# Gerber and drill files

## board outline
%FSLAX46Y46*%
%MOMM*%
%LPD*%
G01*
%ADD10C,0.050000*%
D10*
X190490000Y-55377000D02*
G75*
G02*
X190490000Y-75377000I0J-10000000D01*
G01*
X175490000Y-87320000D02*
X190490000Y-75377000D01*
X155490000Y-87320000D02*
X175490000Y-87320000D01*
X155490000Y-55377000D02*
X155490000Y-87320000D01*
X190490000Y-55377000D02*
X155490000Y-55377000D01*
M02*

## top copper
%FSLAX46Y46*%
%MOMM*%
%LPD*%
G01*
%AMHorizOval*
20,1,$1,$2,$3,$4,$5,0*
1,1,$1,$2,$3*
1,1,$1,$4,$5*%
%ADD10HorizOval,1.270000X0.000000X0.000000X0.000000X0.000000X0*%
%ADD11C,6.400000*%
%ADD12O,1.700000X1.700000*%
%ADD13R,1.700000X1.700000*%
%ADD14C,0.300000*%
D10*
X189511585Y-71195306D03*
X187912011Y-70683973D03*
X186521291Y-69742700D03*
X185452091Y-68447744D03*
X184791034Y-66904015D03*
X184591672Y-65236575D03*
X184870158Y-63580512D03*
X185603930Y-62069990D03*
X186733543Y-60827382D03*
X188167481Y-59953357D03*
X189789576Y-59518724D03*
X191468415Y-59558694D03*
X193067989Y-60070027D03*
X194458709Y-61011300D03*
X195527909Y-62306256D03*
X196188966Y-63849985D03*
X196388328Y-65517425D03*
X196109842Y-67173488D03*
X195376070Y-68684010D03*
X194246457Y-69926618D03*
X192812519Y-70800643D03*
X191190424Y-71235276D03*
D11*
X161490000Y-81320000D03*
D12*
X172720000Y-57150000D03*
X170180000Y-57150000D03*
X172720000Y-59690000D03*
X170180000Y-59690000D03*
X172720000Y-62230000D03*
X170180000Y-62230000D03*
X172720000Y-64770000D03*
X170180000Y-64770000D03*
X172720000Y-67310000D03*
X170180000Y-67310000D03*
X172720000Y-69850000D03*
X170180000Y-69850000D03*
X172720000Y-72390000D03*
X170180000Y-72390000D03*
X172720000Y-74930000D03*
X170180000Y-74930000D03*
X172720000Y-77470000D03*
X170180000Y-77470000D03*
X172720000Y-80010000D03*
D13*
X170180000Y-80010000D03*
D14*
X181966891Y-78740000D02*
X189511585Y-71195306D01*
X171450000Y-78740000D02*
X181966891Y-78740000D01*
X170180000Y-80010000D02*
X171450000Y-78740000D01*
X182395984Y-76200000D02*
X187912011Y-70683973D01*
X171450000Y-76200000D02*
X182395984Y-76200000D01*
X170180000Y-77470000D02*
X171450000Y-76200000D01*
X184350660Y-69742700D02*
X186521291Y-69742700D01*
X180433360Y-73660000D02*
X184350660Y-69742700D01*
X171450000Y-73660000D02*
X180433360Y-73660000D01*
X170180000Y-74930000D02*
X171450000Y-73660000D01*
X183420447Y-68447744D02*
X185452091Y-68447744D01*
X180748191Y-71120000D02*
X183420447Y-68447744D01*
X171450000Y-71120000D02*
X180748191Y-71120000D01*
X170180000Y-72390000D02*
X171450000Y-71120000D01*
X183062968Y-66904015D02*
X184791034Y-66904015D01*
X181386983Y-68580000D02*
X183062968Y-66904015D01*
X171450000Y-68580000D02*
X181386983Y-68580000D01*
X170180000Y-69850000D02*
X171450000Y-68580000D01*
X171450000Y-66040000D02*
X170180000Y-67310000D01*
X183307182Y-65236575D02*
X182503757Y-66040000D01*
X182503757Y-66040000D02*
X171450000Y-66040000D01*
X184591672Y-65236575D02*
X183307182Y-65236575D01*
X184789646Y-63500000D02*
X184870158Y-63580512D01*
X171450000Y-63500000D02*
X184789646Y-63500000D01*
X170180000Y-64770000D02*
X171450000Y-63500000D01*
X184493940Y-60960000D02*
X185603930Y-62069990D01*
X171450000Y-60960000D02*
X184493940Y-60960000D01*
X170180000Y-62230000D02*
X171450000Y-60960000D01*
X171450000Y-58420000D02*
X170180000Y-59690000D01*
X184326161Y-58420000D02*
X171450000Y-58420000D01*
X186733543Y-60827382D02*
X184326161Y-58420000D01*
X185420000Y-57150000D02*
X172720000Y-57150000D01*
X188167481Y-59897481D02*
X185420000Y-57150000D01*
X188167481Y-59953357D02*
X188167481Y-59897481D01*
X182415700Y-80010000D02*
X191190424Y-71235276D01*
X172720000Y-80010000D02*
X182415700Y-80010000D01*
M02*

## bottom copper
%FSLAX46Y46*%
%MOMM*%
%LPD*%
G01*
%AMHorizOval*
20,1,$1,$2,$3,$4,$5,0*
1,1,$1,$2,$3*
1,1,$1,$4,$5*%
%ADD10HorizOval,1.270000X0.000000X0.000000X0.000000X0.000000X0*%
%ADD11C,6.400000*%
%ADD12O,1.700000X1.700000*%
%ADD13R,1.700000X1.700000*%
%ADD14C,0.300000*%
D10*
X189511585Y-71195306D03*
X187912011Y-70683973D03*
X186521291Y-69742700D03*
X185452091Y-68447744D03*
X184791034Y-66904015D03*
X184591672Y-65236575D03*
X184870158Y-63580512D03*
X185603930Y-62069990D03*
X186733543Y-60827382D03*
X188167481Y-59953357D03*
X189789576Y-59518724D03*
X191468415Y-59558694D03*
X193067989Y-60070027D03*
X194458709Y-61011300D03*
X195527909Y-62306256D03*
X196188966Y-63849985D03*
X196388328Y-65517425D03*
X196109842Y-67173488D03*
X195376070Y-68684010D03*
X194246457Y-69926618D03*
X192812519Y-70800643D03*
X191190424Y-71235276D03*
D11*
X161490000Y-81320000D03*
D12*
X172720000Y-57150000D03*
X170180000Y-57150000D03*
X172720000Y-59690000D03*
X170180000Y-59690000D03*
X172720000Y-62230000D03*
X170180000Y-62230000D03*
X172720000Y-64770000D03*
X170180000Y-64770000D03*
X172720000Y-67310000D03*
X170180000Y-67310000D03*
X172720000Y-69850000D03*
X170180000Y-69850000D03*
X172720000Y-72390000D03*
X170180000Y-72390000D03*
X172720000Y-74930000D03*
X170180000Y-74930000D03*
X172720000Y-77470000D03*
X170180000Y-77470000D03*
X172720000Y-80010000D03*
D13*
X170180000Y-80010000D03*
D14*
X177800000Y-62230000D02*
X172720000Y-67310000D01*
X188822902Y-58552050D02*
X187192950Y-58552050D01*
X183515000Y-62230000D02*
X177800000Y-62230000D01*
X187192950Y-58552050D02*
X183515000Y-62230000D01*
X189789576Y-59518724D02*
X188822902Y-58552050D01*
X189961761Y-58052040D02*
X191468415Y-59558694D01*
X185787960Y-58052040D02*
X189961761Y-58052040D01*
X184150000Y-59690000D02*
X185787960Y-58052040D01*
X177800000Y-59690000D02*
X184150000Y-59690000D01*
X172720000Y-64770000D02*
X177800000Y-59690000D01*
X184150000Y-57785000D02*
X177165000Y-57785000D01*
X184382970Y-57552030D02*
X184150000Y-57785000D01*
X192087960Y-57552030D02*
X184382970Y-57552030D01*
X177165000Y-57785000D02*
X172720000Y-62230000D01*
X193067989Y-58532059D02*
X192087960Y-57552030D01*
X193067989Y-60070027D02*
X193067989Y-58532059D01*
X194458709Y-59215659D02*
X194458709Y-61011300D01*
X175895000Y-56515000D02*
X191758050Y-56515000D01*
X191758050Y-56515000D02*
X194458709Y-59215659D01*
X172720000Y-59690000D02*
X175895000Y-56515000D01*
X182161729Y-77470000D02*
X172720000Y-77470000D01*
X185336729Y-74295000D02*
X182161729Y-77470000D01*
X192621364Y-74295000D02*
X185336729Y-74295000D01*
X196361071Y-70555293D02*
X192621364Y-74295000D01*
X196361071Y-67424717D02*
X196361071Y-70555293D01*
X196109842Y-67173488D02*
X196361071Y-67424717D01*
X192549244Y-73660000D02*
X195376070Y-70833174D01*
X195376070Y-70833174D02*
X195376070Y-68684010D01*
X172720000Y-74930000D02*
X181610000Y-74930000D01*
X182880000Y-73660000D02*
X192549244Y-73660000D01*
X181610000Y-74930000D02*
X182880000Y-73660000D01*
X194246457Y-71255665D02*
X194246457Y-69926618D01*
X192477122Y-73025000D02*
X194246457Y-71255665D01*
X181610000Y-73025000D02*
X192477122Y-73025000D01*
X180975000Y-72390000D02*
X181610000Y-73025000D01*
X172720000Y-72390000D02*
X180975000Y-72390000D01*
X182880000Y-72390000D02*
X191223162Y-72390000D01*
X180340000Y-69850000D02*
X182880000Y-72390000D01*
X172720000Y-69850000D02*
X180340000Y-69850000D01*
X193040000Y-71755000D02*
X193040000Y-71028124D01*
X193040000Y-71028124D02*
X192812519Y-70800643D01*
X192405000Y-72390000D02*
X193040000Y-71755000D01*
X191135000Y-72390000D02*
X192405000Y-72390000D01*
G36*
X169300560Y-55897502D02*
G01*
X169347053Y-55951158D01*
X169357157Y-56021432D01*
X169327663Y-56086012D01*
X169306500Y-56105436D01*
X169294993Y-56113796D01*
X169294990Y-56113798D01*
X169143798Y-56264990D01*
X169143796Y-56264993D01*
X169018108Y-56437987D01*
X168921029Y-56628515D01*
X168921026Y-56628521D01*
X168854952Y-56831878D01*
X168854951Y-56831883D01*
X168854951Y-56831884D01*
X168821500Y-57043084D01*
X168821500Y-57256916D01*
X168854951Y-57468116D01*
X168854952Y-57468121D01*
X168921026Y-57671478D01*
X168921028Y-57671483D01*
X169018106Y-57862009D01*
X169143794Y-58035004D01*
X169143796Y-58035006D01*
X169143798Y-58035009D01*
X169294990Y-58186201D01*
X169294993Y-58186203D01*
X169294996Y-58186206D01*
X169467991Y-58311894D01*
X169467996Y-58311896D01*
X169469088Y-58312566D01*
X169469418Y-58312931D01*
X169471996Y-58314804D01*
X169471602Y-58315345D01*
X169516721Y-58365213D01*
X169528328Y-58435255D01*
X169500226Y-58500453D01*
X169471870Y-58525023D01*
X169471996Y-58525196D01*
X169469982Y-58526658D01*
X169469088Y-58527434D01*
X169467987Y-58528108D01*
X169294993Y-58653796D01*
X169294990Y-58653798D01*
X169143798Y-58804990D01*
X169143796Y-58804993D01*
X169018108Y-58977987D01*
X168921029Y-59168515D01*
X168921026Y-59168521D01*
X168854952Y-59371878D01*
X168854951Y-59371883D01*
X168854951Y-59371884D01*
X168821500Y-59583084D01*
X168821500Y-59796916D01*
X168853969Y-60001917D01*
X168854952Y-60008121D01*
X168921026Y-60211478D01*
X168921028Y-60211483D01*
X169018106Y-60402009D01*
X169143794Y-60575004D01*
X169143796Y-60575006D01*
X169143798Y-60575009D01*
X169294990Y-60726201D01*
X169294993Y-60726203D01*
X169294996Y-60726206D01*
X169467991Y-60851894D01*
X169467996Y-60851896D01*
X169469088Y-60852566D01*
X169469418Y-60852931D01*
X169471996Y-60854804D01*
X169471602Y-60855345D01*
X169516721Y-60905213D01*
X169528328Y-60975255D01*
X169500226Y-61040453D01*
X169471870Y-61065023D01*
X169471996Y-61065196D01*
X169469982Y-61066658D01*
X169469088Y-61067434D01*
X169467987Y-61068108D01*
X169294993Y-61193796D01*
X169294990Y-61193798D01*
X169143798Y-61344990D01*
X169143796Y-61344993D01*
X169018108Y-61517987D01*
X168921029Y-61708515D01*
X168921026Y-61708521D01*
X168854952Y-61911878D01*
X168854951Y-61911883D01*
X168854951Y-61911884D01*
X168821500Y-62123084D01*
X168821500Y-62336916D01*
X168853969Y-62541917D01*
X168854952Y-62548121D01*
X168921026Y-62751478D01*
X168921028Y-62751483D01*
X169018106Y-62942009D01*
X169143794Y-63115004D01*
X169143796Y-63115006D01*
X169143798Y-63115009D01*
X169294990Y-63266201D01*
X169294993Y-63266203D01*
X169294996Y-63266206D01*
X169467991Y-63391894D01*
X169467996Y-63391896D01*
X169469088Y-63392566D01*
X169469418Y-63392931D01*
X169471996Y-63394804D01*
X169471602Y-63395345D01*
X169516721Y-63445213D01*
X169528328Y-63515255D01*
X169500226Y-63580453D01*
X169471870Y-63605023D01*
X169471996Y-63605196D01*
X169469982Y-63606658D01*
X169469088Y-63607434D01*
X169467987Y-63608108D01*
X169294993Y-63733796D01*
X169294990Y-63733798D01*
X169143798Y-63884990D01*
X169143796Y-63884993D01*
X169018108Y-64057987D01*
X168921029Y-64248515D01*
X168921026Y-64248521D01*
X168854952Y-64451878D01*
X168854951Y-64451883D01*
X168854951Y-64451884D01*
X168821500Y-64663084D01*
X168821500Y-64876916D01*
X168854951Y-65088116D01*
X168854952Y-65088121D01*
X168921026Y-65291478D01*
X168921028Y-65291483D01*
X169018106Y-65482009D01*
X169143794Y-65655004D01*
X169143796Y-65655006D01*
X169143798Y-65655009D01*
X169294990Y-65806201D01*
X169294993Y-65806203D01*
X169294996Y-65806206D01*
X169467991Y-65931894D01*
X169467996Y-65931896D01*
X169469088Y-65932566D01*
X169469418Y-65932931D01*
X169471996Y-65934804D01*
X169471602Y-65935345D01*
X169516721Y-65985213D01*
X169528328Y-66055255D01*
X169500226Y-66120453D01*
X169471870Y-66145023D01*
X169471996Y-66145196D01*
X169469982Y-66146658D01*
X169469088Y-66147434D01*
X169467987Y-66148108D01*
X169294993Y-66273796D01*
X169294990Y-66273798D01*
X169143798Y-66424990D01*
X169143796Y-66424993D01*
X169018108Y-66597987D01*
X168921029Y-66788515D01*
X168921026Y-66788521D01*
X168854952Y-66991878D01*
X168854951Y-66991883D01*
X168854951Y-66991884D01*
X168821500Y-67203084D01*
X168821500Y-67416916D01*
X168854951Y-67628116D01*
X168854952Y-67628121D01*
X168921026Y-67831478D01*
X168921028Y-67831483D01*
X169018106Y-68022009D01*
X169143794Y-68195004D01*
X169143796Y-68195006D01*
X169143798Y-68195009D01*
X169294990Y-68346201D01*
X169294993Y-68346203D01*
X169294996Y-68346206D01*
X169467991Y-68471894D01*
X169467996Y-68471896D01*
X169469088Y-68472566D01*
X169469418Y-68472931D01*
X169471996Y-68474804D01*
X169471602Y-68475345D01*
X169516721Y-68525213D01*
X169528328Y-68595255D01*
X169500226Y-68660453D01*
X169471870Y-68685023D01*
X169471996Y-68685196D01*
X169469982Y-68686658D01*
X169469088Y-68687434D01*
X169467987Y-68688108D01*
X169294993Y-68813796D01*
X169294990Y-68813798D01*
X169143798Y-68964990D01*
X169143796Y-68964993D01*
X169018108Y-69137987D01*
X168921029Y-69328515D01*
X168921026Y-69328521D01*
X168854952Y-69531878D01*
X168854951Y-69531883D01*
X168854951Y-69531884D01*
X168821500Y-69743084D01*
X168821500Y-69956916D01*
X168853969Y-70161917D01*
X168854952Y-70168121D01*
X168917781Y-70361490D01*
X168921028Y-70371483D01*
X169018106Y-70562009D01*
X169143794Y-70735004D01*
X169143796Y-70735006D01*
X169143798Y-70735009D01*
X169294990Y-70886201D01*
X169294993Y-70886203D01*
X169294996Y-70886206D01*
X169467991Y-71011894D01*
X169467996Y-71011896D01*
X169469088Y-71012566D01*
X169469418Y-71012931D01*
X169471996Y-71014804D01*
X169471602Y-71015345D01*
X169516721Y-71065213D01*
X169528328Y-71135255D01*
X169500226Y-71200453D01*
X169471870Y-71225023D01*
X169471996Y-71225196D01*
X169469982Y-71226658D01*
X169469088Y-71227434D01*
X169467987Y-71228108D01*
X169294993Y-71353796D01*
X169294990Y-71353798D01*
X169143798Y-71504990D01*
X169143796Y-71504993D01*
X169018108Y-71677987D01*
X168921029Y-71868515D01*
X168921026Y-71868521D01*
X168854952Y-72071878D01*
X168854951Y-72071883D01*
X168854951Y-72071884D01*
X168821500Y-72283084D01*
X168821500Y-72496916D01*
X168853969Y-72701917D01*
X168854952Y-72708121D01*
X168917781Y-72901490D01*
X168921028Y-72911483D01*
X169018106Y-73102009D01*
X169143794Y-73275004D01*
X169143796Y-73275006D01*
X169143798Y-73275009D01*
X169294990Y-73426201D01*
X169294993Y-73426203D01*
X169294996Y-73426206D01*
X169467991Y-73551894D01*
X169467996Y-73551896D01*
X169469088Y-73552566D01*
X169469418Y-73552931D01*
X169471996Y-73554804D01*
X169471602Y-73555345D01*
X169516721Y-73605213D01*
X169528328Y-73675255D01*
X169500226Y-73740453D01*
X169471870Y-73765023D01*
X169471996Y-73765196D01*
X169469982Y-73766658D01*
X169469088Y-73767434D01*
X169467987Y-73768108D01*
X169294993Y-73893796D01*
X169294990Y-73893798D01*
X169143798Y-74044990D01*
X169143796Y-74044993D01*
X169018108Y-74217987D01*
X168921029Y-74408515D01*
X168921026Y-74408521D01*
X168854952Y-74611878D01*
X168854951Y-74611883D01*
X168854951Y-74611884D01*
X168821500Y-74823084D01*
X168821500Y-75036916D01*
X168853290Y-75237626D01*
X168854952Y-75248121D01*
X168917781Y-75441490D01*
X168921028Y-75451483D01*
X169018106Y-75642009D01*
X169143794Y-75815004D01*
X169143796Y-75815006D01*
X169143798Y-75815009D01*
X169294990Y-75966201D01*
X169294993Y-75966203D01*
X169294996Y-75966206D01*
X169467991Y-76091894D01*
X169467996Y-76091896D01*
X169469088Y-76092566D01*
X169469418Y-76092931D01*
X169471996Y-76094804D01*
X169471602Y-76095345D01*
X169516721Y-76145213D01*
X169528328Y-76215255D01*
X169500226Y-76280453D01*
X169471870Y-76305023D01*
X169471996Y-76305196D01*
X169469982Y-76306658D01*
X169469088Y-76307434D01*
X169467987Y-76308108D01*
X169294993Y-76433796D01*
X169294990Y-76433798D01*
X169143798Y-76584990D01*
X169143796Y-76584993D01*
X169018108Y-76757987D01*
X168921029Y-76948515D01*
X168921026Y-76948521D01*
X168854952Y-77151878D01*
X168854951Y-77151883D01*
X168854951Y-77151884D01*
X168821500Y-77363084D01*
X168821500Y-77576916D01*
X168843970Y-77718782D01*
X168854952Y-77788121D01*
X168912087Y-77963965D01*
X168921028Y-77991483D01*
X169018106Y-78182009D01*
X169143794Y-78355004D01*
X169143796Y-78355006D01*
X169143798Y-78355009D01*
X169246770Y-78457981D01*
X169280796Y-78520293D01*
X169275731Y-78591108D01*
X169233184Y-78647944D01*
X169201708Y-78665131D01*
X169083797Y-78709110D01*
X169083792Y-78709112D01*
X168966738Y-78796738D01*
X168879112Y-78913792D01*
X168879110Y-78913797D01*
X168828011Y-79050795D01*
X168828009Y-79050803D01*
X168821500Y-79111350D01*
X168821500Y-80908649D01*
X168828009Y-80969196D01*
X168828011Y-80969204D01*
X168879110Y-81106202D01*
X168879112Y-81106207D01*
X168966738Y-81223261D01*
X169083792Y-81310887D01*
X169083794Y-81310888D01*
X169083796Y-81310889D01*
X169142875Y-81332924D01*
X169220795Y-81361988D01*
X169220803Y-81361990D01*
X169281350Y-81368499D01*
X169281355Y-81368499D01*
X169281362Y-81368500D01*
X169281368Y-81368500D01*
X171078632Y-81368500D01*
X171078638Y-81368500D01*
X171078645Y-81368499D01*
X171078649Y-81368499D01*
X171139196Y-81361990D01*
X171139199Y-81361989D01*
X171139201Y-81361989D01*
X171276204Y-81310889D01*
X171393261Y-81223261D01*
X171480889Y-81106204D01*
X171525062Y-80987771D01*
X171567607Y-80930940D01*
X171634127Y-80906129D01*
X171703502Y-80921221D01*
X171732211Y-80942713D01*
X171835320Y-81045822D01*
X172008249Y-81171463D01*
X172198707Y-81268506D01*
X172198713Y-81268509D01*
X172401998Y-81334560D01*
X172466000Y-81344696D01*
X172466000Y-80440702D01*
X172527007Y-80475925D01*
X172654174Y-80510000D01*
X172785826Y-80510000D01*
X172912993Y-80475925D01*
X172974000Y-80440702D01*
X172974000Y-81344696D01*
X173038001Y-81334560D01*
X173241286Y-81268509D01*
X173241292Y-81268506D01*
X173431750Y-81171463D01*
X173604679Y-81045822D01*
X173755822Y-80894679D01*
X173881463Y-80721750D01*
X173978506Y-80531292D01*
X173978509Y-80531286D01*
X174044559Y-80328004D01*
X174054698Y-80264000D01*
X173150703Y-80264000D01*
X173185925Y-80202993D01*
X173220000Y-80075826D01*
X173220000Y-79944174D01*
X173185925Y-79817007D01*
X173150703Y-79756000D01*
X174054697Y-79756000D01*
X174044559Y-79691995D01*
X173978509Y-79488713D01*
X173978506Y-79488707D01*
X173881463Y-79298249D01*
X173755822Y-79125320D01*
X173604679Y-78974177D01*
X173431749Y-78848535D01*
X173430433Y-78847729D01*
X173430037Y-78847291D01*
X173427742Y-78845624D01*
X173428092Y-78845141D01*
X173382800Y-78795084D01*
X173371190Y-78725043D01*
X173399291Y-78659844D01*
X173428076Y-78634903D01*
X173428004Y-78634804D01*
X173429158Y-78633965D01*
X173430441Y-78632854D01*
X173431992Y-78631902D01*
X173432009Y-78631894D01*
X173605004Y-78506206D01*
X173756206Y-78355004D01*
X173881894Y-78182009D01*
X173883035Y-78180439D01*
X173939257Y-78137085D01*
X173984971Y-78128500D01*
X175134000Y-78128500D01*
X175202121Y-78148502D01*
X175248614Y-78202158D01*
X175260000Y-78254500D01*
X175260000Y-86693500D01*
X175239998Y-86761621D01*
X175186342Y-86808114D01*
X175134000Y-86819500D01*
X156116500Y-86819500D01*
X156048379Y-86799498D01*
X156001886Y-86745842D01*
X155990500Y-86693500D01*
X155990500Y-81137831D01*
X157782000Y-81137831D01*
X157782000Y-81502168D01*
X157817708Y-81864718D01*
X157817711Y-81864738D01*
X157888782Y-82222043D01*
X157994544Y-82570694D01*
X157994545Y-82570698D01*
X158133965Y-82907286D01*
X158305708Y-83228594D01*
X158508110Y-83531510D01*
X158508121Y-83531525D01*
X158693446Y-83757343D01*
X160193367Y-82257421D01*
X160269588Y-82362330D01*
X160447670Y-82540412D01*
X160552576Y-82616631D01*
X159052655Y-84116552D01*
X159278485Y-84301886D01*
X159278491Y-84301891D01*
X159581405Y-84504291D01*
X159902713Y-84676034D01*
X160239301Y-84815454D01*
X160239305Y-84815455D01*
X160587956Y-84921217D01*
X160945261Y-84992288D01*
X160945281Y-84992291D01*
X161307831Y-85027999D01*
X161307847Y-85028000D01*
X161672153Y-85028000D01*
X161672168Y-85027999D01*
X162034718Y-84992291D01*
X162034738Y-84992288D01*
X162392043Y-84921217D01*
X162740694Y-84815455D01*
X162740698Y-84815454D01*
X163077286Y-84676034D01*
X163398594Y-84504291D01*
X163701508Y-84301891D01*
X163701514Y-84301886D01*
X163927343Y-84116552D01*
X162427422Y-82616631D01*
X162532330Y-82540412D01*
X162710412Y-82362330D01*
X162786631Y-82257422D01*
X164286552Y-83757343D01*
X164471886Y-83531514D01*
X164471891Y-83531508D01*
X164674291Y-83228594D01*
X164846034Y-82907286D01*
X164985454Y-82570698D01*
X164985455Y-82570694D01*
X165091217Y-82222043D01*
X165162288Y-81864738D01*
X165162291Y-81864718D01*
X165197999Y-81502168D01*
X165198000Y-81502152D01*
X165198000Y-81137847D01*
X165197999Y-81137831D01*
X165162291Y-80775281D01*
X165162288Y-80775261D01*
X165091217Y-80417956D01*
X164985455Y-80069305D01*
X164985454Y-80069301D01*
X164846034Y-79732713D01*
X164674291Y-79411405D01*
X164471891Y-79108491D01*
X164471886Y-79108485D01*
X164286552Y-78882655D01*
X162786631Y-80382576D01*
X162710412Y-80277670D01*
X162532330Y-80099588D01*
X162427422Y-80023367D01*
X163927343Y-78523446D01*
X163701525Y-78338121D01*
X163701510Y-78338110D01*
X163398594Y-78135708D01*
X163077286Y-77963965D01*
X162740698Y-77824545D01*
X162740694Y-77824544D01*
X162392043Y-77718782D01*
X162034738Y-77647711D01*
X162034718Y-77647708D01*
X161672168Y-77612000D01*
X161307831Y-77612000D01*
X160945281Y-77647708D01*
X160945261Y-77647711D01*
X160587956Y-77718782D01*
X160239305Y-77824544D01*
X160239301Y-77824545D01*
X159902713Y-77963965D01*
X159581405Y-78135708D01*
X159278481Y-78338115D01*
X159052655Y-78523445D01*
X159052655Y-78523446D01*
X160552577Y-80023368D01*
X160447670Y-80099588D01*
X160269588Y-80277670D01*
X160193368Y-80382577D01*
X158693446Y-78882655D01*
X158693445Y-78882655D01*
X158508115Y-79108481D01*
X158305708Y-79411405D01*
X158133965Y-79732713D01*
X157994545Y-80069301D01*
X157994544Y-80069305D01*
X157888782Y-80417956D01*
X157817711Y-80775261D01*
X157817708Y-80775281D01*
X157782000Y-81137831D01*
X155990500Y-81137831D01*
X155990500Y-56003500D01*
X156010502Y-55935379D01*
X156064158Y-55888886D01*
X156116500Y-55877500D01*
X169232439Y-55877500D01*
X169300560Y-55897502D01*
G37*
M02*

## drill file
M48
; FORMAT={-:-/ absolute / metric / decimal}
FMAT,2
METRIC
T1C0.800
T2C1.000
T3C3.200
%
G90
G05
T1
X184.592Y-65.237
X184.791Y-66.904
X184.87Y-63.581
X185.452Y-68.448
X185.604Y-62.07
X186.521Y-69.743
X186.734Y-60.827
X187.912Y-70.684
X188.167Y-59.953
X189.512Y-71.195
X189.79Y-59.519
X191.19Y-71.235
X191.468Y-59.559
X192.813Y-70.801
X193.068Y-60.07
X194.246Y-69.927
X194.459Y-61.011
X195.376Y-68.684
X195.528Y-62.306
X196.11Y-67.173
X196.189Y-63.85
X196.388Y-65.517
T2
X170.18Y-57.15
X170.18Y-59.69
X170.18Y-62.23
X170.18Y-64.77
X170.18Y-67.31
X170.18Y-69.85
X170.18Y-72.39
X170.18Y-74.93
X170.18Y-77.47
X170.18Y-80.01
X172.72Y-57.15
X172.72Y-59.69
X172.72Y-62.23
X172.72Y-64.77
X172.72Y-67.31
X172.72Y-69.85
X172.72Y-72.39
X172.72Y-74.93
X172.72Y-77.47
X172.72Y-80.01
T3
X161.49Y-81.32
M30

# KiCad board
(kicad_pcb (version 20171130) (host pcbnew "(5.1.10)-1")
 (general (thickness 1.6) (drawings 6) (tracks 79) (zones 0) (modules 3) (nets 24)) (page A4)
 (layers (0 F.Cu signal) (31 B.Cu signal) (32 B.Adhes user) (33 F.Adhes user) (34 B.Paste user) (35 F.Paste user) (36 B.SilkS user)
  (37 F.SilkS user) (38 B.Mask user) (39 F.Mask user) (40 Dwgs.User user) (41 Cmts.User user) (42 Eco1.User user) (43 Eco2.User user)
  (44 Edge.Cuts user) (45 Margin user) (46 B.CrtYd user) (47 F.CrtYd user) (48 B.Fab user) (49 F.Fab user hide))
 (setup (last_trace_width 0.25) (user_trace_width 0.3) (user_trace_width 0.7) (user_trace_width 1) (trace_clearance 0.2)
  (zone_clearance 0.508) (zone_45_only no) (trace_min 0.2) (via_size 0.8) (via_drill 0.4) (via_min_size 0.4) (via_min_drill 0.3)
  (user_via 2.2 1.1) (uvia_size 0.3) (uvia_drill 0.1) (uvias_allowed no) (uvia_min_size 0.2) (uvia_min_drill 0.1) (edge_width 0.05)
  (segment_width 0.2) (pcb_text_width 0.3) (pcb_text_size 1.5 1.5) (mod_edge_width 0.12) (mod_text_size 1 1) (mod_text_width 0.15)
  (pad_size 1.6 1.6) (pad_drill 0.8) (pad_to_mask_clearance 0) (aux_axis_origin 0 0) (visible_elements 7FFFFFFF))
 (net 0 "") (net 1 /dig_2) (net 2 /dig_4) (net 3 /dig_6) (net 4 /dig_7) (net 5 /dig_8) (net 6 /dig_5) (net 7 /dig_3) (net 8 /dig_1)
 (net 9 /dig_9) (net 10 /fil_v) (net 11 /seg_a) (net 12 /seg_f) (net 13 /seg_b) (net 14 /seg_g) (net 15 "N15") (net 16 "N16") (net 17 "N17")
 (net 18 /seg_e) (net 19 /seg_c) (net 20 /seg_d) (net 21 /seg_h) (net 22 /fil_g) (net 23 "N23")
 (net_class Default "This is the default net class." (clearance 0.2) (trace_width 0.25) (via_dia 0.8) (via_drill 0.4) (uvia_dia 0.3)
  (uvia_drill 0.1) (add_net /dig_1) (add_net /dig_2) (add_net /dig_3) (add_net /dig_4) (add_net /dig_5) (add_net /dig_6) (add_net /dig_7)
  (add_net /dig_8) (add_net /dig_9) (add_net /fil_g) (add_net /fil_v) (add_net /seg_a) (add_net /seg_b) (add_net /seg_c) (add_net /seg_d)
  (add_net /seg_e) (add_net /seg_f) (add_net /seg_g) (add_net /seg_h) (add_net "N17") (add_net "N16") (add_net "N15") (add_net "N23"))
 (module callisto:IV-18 (layer F.Cu) (at 190.49 65.377 15)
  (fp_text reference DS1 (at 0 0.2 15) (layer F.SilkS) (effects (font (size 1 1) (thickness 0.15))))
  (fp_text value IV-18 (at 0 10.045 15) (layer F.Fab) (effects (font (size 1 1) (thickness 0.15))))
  (pad 22 thru_hole oval (at -2.450965 5.36682 15) (size 1.27 1.27) (drill 0.8) (layers *.Cu *.Mask) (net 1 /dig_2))
  (pad 21 thru_hole oval (at -3.863692 4.45891 15) (size 1.27 1.27) (drill 0.8) (layers *.Cu *.Mask) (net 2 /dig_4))
  (pad 20 thru_hole oval (at -4.963405 3.189765 15) (size 1.27 1.27) (drill 0.8) (layers *.Cu *.Mask) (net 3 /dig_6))
  (pad 19 thru_hole oval (at -5.661013 1.662204 15) (size 1.27 1.27) (drill 0.8) (layers *.Cu *.Mask) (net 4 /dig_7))
  (pad 18 thru_hole oval (at -5.899999 -0.000018 15) (size 1.27 1.27) (drill 0.8) (layers *.Cu *.Mask) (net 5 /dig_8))
  (pad 17 thru_hole oval (at -5.661003 -1.66224 15) (size 1.27 1.27) (drill 0.8) (layers *.Cu *.Mask) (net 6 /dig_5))
  (pad 16 thru_hole oval (at -4.963385 -3.189796 15) (size 1.27 1.27) (drill 0.8) (layers *.Cu *.Mask) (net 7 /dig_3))
  (pad 15 thru_hole oval (at -3.863664 -4.458934 15) (size 1.27 1.27) (drill 0.8) (layers *.Cu *.Mask) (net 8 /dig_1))
  (pad 14 thru_hole oval (at -2.450931 -5.366836 15) (size 1.27 1.27) (drill 0.8) (layers *.Cu *.Mask) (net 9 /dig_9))
  (pad 13 thru_hole oval (at -0.839639 -5.839949 15) (size 1.27 1.27) (drill 0.8) (layers *.Cu *.Mask) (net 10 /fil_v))
  (pad 12 thru_hole oval (at 0.839676 -5.839943 15) (size 1.27 1.27) (drill 0.8) (layers *.Cu *.Mask) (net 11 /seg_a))
  (pad 11 thru_hole oval (at 2.450965 -5.36682 15) (size 1.27 1.27) (drill 0.8) (layers *.Cu *.Mask) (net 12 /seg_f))
  (pad 10 thru_hole oval (at 3.863692 -4.45891 15) (size 1.27 1.27) (drill 0.8) (layers *.Cu *.Mask) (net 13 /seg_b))
  (pad 9 thru_hole oval (at 4.963405 -3.189765 15) (size 1.27 1.27) (drill 0.8) (layers *.Cu *.Mask) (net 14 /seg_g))
  (pad 8 thru_hole oval (at 5.661013 -1.662204 15) (size 1.27 1.27) (drill 0.8) (layers *.Cu *.Mask) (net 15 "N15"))
  (pad 7 thru_hole oval (at 5.899999 0.000018 15) (size 1.27 1.27) (drill 0.8) (layers *.Cu *.Mask) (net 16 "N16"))
  (pad 6 thru_hole oval (at 5.661003 1.66224 15) (size 1.27 1.27) (drill 0.8) (layers *.Cu *.Mask) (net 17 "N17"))
  (pad 5 thru_hole oval (at 4.963385 3.189796 15) (size 1.27 1.27) (drill 0.8) (layers *.Cu *.Mask) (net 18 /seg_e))
  (pad 4 thru_hole oval (at 3.863664 4.458934 15) (size 1.27 1.27) (drill 0.8) (layers *.Cu *.Mask) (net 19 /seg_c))
  (pad 3 thru_hole oval (at 2.450931 5.366836 15) (size 1.27 1.27) (drill 0.8) (layers *.Cu *.Mask) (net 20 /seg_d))
  (pad 2 thru_hole oval (at 0.839639 5.839949 15) (size 1.27 1.27) (drill 0.8) (layers *.Cu *.Mask) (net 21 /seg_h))
  (pad 1 thru_hole oval (at -0.839676 5.839943 15) (size 1.27 1.27) (drill 0.8) (layers *.Cu *.Mask) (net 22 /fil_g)))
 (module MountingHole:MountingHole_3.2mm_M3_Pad (layer F.Cu) (at 161.49 81.32)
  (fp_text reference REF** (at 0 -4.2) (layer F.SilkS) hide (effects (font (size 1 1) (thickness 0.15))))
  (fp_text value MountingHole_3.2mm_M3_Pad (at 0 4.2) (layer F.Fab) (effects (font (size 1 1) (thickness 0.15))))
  (pad 1 thru_hole circle (at 0 0) (size 6.4 6.4) (drill 3.2) (layers *.Cu *.Mask) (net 22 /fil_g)))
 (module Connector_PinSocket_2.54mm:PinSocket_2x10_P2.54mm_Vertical (layer F.Cu) (at 170.18 80.01 180)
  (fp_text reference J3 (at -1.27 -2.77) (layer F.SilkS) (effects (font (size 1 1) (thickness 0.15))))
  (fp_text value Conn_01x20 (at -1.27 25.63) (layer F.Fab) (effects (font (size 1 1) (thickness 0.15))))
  (pad 20 thru_hole oval (at -2.54 22.86 180) (size 1.7 1.7) (drill 1) (layers *.Cu *.Mask) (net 10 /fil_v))
  (pad 19 thru_hole oval (at 0 22.86 180) (size 1.7 1.7) (drill 1) (layers *.Cu *.Mask) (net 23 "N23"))
  (pad 18 thru_hole oval (at -2.54 20.32 180) (size 1.7 1.7) (drill 1) (layers *.Cu *.Mask) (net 14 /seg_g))
  (pad 17 thru_hole oval (at 0 20.32 180) (size 1.7 1.7) (drill 1) (layers *.Cu *.Mask) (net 9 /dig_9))
  (pad 16 thru_hole oval (at -2.54 17.78 180) (size 1.7 1.7) (drill 1) (layers *.Cu *.Mask) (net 13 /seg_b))
  (pad 15 thru_hole oval (at 0 17.78 180) (size 1.7 1.7) (drill 1) (layers *.Cu *.Mask) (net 8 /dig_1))
  (pad 14 thru_hole oval (at -2.54 15.24 180) (size 1.7 1.7) (drill 1) (layers *.Cu *.Mask) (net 12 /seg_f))
  (pad 13 thru_hole oval (at 0 15.24 180) (size 1.7 1.7) (drill 1) (layers *.Cu *.Mask) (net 7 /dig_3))
  (pad 12 thru_hole oval (at -2.54 12.7 180) (size 1.7 1.7) (drill 1) (layers *.Cu *.Mask) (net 11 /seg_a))
  (pad 11 thru_hole oval (at 0 12.7 180) (size 1.7 1.7) (drill 1) (layers *.Cu *.Mask) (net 6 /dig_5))
  (pad 10 thru_hole oval (at -2.54 10.16 180) (size 1.7 1.7) (drill 1) (layers *.Cu *.Mask) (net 21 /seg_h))
  (pad 9 thru_hole oval (at 0 10.16 180) (size 1.7 1.7) (drill 1) (layers *.Cu *.Mask) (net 5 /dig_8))
  (pad 8 thru_hole oval (at -2.54 7.62 180) (size 1.7 1.7) (drill 1) (layers *.Cu *.Mask) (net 20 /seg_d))
  (pad 7 thru_hole oval (at 0 7.62 180) (size 1.7 1.7) (drill 1) (layers *.Cu *.Mask) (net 4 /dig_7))
  (pad 6 thru_hole oval (at -2.54 5.08 180) (size 1.7 1.7) (drill 1) (layers *.Cu *.Mask) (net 19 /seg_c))
  (pad 5 thru_hole oval (at 0 5.08 180) (size 1.7 1.7) (drill 1) (layers *.Cu *.Mask) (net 3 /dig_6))
  (pad 4 thru_hole oval (at -2.54 2.54 180) (size 1.7 1.7) (drill 1) (layers *.Cu *.Mask) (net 18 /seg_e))
  (pad 3 thru_hole oval (at 0 2.54 180) (size 1.7 1.7) (drill 1) (layers *.Cu *.Mask) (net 2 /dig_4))
  (pad 2 thru_hole oval (at -2.54 0 180) (size 1.7 1.7) (drill 1) (layers *.Cu *.Mask) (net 22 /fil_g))
  (pad 1 thru_hole rect (at 0 0 180) (size 1.7 1.7) (drill 1) (layers *.Cu *.Mask) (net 1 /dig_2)))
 (gr_arc (start 190.49 65.377) (end 190.49 75.377) (angle -180) (layer Edge.Cuts) (width 0.05))
 (gr_line (start 175.49 87.32) (end 190.49 75.377) (layer Edge.Cuts) (width 0.05))
 (gr_line (start 155.49 87.32) (end 175.49 87.32) (layer Edge.Cuts) (width 0.05))
 (gr_line (start 155.49 55.377) (end 155.49 87.32) (layer Edge.Cuts) (width 0.05))
 (gr_line (start 190.49 55.377) (end 155.49 55.377) (layer Edge.Cuts) (width 0.05))
 (segment (start 181.966891 78.74) (end 189.511585 71.195306) (width 0.3) (layer F.Cu) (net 1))
 (segment (start 171.45 78.74) (end 181.966891 78.74) (width 0.3) (layer F.Cu) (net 1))
 (segment (start 170.18 80.01) (end 171.45 78.74) (width 0.3) (layer F.Cu) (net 1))
 (segment (start 182.395984 76.2) (end 187.912011 70.683973) (width 0.3) (layer F.Cu) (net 2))
 (segment (start 171.45 76.2) (end 182.395984 76.2) (width 0.3) (layer F.Cu) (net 2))
 (segment (start 170.18 77.47) (end 171.45 76.2) (width 0.3) (layer F.Cu) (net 2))
 (segment (start 184.35066 69.7427) (end 186.521291 69.7427) (width 0.3) (layer F.Cu) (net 3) (status 20))
 (segment (start 180.43336 73.66) (end 184.35066 69.7427) (width 0.3) (layer F.Cu) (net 3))
 (segment (start 171.45 73.66) (end 180.43336 73.66) (width 0.3) (layer F.Cu) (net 3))
 (segment (start 170.18 74.93) (end 171.45 73.66) (width 0.3) (layer F.Cu) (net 3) (status 10))
 (segment (start 183.420447 68.447744) (end 185.452091 68.447744) (width 0.3) (layer F.Cu) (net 4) (status 20))
 (segment (start 180.748191 71.12) (end 183.420447 68.447744) (width 0.3) (layer F.Cu) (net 4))
 (segment (start 171.45 71.12) (end 180.748191 71.12) (width 0.3) (layer F.Cu) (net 4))
 (segment (start 170.18 72.39) (end 171.45 71.12) (width 0.3) (layer F.Cu) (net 4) (status 10))
 (segment (start 183.062968 66.904015) (end 184.791034 66.904015) (width 0.3) (layer F.Cu) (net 5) (status 20))
 (segment (start 181.386983 68.58) (end 183.062968 66.904015) (width 0.3) (layer F.Cu) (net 5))
 (segment (start 171.45 68.58) (end 181.386983 68.58) (width 0.3) (layer F.Cu) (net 5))
 (segment (start 170.18 69.85) (end 171.45 68.58) (width 0.3) (layer F.Cu) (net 5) (status 10))
 (segment (start 171.45 66.04) (end 170.18 67.31) (width 0.3) (layer F.Cu) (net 6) (status 20))
 (segment (start 183.307182 65.236575) (end 182.503757 66.04) (width 0.3) (layer F.Cu) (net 6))
 (segment (start 182.503757 66.04) (end 171.45 66.04) (width 0.3) (layer F.Cu) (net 6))
 (segment (start 184.591672 65.236575) (end 183.307182 65.236575) (width 0.3) (layer F.Cu) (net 6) (status 10))
 (segment (start 184.789646 63.5) (end 184.870158 63.580512) (width 0.3) (layer F.Cu) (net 7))
 (segment (start 171.45 63.5) (end 184.789646 63.5) (width 0.3) (layer F.Cu) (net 7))
 (segment (start 170.18 64.77) (end 171.45 63.5) (width 0.3) (layer F.Cu) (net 7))
 (segment (start 184.49394 60.96) (end 185.60393 62.06999) (width 0.3) (layer F.Cu) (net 8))
 (segment (start 171.45 60.96) (end 184.49394 60.96) (width 0.3) (layer F.Cu) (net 8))
 (segment (start 170.18 62.23) (end 171.45 60.96) (width 0.3) (layer F.Cu) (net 8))
 (segment (start 171.45 58.42) (end 170.18 59.69) (width 0.3) (layer F.Cu) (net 9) (status 20))
 (segment (start 184.326161 58.42) (end 171.45 58.42) (width 0.3) (layer F.Cu) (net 9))
 (segment (start 186.733543 60.827382) (end 184.326161 58.42) (width 0.3) (layer F.Cu) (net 9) (status 10))
 (segment (start 185.42 57.15) (end 172.72 57.15) (width 0.3) (layer F.Cu) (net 10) (status 20))
 (segment (start 188.167481 59.897481) (end 185.42 57.15) (width 0.3) (layer F.Cu) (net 10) (status 10))
 (segment (start 188.167481 59.953357) (end 188.167481 59.897481) (width 0.3) (layer F.Cu) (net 10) (status 30))
 (segment (start 177.8 62.23) (end 172.72 67.31) (width 0.3) (layer B.Cu) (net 11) (status 20))
 (segment (start 188.822902 58.55205) (end 187.19295 58.55205) (width 0.3) (layer B.Cu) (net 11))
 (segment (start 183.515 62.23) (end 177.8 62.23) (width 0.3) (layer B.Cu) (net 11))
 (segment (start 187.19295 58.55205) (end 183.515 62.23) (width 0.3) (layer B.Cu) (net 11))
 (segment (start 189.789576 59.518724) (end 188.822902 58.55205) (width 0.3) (layer B.Cu) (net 11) (status 10))
 (segment (start 189.961761 58.05204) (end 191.468415 59.558694) (width 0.3) (layer B.Cu) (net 12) (status 20))
 (segment (start 185.78796 58.05204) (end 189.961761 58.05204) (width 0.3) (layer B.Cu) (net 12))
 (segment (start 184.15 59.69) (end 185.78796 58.05204) (width 0.3) (layer B.Cu) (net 12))
 (segment (start 177.8 59.69) (end 184.15 59.69) (width 0.3) (layer B.Cu) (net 12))
 (segment (start 172.72 64.77) (end 177.8 59.69) (width 0.3) (layer B.Cu) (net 12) (status 10))
 (segment (start 184.15 57.785) (end 177.165 57.785) (width 0.3) (layer B.Cu) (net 13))
 (segment (start 184.38297 57.55203) (end 184.15 57.785) (width 0.3) (layer B.Cu) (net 13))
 (segment (start 192.08796 57.55203) (end 184.38297 57.55203) (width 0.3) (layer B.Cu) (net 13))
 (segment (start 177.165 57.785) (end 172.72 62.23) (width 0.3) (layer B.Cu) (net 13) (status 20))
 (segment (start 193.067989 58.532059) (end 192.08796 57.55203) (width 0.3) (layer B.Cu) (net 13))
 (segment (start 193.067989 60.070027) (end 193.067989 58.532059) (width 0.3) (layer B.Cu) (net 13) (status 10))
 (segment (start 194.458709 59.215659) (end 194.458709 61.0113) (width 0.3) (layer B.Cu) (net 14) (status 20))
 (segment (start 175.895 56.515) (end 191.75805 56.515) (width 0.3) (layer B.Cu) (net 14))
 (segment (start 191.75805 56.515) (end 194.458709 59.215659) (width 0.3) (layer B.Cu) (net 14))
 (segment (start 172.72 59.69) (end 175.895 56.515) (width 0.3) (layer B.Cu) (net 14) (status 10))
 (segment (start 182.161729 77.47) (end 172.72 77.47) (width 0.3) (layer B.Cu) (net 18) (status 20))
 (segment (start 185.336729 74.295) (end 182.161729 77.47) (width 0.3) (layer B.Cu) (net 18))
 (segment (start 192.621364 74.295) (end 185.336729 74.295) (width 0.3) (layer B.Cu) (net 18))
 (segment (start 196.361071 70.555293) (end 192.621364 74.295) (width 0.3) (layer B.Cu) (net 18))
 (segment (start 196.361071 67.424717) (end 196.361071 70.555293) (width 0.3) (layer B.Cu) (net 18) (status 10))
 (segment (start 196.109842 67.173488) (end 196.361071 67.424717) (width 0.3) (layer B.Cu) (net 18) (status 30))
 (segment (start 192.549244 73.66) (end 195.37607 70.833174) (width 0.3) (layer B.Cu) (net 19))
 (segment (start 195.37607 70.833174) (end 195.37607 68.68401) (width 0.3) (layer B.Cu) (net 19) (status 20))
 (segment (start 172.72 74.93) (end 181.61 74.93) (width 0.3) (layer B.Cu) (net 19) (status 10))
 (segment (start 182.88 73.66) (end 192.549244 73.66) (width 0.3) (layer B.Cu) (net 19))
 (segment (start 181.61 74.93) (end 182.88 73.66) (width 0.3) (layer B.Cu) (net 19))
 (segment (start 194.246457 71.255665) (end 194.246457 69.926618) (width 0.3) (layer B.Cu) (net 20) (status 20))
 (segment (start 192.477122 73.025) (end 194.246457 71.255665) (width 0.3) (layer B.Cu) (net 20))
 (segment (start 181.61 73.025) (end 192.477122 73.025) (width 0.3) (layer B.Cu) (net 20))
 (segment (start 180.975 72.39) (end 181.61 73.025) (width 0.3) (layer B.Cu) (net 20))
 (segment (start 172.72 72.39) (end 180.975 72.39) (width 0.3) (layer B.Cu) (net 20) (status 10))
 (segment (start 182.88 72.39) (end 191.223162 72.39) (width 0.3) (layer B.Cu) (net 21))
 (segment (start 180.34 69.85) (end 182.88 72.39) (width 0.3) (layer B.Cu) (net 21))
 (segment (start 172.72 69.85) (end 180.34 69.85) (width 0.3) (layer B.Cu) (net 21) (status 10))
 (segment (start 193.04 71.755) (end 193.04 71.028124) (width 0.3) (layer B.Cu) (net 21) (status 20))
 (segment (start 193.04 71.028124) (end 192.812519 70.800643) (width 0.3) (layer B.Cu) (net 21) (status 30))
 (segment (start 192.405 72.39) (end 193.04 71.755) (width 0.3) (layer B.Cu) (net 21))
 (segment (start 191.135 72.39) (end 192.405 72.39) (width 0.3) (layer B.Cu) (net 21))
 (segment (start 182.4157 80.01) (end 191.190424 71.235276) (width 0.3) (layer F.Cu) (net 22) (status 20))
 (segment (start 172.72 80.01) (end 182.4157 80.01) (width 0.3) (layer F.Cu) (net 22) (status 10))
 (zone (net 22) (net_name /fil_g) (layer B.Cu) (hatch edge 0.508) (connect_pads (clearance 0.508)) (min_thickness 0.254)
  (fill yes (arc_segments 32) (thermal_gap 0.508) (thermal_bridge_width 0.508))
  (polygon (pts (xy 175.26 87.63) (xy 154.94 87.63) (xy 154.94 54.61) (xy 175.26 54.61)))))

